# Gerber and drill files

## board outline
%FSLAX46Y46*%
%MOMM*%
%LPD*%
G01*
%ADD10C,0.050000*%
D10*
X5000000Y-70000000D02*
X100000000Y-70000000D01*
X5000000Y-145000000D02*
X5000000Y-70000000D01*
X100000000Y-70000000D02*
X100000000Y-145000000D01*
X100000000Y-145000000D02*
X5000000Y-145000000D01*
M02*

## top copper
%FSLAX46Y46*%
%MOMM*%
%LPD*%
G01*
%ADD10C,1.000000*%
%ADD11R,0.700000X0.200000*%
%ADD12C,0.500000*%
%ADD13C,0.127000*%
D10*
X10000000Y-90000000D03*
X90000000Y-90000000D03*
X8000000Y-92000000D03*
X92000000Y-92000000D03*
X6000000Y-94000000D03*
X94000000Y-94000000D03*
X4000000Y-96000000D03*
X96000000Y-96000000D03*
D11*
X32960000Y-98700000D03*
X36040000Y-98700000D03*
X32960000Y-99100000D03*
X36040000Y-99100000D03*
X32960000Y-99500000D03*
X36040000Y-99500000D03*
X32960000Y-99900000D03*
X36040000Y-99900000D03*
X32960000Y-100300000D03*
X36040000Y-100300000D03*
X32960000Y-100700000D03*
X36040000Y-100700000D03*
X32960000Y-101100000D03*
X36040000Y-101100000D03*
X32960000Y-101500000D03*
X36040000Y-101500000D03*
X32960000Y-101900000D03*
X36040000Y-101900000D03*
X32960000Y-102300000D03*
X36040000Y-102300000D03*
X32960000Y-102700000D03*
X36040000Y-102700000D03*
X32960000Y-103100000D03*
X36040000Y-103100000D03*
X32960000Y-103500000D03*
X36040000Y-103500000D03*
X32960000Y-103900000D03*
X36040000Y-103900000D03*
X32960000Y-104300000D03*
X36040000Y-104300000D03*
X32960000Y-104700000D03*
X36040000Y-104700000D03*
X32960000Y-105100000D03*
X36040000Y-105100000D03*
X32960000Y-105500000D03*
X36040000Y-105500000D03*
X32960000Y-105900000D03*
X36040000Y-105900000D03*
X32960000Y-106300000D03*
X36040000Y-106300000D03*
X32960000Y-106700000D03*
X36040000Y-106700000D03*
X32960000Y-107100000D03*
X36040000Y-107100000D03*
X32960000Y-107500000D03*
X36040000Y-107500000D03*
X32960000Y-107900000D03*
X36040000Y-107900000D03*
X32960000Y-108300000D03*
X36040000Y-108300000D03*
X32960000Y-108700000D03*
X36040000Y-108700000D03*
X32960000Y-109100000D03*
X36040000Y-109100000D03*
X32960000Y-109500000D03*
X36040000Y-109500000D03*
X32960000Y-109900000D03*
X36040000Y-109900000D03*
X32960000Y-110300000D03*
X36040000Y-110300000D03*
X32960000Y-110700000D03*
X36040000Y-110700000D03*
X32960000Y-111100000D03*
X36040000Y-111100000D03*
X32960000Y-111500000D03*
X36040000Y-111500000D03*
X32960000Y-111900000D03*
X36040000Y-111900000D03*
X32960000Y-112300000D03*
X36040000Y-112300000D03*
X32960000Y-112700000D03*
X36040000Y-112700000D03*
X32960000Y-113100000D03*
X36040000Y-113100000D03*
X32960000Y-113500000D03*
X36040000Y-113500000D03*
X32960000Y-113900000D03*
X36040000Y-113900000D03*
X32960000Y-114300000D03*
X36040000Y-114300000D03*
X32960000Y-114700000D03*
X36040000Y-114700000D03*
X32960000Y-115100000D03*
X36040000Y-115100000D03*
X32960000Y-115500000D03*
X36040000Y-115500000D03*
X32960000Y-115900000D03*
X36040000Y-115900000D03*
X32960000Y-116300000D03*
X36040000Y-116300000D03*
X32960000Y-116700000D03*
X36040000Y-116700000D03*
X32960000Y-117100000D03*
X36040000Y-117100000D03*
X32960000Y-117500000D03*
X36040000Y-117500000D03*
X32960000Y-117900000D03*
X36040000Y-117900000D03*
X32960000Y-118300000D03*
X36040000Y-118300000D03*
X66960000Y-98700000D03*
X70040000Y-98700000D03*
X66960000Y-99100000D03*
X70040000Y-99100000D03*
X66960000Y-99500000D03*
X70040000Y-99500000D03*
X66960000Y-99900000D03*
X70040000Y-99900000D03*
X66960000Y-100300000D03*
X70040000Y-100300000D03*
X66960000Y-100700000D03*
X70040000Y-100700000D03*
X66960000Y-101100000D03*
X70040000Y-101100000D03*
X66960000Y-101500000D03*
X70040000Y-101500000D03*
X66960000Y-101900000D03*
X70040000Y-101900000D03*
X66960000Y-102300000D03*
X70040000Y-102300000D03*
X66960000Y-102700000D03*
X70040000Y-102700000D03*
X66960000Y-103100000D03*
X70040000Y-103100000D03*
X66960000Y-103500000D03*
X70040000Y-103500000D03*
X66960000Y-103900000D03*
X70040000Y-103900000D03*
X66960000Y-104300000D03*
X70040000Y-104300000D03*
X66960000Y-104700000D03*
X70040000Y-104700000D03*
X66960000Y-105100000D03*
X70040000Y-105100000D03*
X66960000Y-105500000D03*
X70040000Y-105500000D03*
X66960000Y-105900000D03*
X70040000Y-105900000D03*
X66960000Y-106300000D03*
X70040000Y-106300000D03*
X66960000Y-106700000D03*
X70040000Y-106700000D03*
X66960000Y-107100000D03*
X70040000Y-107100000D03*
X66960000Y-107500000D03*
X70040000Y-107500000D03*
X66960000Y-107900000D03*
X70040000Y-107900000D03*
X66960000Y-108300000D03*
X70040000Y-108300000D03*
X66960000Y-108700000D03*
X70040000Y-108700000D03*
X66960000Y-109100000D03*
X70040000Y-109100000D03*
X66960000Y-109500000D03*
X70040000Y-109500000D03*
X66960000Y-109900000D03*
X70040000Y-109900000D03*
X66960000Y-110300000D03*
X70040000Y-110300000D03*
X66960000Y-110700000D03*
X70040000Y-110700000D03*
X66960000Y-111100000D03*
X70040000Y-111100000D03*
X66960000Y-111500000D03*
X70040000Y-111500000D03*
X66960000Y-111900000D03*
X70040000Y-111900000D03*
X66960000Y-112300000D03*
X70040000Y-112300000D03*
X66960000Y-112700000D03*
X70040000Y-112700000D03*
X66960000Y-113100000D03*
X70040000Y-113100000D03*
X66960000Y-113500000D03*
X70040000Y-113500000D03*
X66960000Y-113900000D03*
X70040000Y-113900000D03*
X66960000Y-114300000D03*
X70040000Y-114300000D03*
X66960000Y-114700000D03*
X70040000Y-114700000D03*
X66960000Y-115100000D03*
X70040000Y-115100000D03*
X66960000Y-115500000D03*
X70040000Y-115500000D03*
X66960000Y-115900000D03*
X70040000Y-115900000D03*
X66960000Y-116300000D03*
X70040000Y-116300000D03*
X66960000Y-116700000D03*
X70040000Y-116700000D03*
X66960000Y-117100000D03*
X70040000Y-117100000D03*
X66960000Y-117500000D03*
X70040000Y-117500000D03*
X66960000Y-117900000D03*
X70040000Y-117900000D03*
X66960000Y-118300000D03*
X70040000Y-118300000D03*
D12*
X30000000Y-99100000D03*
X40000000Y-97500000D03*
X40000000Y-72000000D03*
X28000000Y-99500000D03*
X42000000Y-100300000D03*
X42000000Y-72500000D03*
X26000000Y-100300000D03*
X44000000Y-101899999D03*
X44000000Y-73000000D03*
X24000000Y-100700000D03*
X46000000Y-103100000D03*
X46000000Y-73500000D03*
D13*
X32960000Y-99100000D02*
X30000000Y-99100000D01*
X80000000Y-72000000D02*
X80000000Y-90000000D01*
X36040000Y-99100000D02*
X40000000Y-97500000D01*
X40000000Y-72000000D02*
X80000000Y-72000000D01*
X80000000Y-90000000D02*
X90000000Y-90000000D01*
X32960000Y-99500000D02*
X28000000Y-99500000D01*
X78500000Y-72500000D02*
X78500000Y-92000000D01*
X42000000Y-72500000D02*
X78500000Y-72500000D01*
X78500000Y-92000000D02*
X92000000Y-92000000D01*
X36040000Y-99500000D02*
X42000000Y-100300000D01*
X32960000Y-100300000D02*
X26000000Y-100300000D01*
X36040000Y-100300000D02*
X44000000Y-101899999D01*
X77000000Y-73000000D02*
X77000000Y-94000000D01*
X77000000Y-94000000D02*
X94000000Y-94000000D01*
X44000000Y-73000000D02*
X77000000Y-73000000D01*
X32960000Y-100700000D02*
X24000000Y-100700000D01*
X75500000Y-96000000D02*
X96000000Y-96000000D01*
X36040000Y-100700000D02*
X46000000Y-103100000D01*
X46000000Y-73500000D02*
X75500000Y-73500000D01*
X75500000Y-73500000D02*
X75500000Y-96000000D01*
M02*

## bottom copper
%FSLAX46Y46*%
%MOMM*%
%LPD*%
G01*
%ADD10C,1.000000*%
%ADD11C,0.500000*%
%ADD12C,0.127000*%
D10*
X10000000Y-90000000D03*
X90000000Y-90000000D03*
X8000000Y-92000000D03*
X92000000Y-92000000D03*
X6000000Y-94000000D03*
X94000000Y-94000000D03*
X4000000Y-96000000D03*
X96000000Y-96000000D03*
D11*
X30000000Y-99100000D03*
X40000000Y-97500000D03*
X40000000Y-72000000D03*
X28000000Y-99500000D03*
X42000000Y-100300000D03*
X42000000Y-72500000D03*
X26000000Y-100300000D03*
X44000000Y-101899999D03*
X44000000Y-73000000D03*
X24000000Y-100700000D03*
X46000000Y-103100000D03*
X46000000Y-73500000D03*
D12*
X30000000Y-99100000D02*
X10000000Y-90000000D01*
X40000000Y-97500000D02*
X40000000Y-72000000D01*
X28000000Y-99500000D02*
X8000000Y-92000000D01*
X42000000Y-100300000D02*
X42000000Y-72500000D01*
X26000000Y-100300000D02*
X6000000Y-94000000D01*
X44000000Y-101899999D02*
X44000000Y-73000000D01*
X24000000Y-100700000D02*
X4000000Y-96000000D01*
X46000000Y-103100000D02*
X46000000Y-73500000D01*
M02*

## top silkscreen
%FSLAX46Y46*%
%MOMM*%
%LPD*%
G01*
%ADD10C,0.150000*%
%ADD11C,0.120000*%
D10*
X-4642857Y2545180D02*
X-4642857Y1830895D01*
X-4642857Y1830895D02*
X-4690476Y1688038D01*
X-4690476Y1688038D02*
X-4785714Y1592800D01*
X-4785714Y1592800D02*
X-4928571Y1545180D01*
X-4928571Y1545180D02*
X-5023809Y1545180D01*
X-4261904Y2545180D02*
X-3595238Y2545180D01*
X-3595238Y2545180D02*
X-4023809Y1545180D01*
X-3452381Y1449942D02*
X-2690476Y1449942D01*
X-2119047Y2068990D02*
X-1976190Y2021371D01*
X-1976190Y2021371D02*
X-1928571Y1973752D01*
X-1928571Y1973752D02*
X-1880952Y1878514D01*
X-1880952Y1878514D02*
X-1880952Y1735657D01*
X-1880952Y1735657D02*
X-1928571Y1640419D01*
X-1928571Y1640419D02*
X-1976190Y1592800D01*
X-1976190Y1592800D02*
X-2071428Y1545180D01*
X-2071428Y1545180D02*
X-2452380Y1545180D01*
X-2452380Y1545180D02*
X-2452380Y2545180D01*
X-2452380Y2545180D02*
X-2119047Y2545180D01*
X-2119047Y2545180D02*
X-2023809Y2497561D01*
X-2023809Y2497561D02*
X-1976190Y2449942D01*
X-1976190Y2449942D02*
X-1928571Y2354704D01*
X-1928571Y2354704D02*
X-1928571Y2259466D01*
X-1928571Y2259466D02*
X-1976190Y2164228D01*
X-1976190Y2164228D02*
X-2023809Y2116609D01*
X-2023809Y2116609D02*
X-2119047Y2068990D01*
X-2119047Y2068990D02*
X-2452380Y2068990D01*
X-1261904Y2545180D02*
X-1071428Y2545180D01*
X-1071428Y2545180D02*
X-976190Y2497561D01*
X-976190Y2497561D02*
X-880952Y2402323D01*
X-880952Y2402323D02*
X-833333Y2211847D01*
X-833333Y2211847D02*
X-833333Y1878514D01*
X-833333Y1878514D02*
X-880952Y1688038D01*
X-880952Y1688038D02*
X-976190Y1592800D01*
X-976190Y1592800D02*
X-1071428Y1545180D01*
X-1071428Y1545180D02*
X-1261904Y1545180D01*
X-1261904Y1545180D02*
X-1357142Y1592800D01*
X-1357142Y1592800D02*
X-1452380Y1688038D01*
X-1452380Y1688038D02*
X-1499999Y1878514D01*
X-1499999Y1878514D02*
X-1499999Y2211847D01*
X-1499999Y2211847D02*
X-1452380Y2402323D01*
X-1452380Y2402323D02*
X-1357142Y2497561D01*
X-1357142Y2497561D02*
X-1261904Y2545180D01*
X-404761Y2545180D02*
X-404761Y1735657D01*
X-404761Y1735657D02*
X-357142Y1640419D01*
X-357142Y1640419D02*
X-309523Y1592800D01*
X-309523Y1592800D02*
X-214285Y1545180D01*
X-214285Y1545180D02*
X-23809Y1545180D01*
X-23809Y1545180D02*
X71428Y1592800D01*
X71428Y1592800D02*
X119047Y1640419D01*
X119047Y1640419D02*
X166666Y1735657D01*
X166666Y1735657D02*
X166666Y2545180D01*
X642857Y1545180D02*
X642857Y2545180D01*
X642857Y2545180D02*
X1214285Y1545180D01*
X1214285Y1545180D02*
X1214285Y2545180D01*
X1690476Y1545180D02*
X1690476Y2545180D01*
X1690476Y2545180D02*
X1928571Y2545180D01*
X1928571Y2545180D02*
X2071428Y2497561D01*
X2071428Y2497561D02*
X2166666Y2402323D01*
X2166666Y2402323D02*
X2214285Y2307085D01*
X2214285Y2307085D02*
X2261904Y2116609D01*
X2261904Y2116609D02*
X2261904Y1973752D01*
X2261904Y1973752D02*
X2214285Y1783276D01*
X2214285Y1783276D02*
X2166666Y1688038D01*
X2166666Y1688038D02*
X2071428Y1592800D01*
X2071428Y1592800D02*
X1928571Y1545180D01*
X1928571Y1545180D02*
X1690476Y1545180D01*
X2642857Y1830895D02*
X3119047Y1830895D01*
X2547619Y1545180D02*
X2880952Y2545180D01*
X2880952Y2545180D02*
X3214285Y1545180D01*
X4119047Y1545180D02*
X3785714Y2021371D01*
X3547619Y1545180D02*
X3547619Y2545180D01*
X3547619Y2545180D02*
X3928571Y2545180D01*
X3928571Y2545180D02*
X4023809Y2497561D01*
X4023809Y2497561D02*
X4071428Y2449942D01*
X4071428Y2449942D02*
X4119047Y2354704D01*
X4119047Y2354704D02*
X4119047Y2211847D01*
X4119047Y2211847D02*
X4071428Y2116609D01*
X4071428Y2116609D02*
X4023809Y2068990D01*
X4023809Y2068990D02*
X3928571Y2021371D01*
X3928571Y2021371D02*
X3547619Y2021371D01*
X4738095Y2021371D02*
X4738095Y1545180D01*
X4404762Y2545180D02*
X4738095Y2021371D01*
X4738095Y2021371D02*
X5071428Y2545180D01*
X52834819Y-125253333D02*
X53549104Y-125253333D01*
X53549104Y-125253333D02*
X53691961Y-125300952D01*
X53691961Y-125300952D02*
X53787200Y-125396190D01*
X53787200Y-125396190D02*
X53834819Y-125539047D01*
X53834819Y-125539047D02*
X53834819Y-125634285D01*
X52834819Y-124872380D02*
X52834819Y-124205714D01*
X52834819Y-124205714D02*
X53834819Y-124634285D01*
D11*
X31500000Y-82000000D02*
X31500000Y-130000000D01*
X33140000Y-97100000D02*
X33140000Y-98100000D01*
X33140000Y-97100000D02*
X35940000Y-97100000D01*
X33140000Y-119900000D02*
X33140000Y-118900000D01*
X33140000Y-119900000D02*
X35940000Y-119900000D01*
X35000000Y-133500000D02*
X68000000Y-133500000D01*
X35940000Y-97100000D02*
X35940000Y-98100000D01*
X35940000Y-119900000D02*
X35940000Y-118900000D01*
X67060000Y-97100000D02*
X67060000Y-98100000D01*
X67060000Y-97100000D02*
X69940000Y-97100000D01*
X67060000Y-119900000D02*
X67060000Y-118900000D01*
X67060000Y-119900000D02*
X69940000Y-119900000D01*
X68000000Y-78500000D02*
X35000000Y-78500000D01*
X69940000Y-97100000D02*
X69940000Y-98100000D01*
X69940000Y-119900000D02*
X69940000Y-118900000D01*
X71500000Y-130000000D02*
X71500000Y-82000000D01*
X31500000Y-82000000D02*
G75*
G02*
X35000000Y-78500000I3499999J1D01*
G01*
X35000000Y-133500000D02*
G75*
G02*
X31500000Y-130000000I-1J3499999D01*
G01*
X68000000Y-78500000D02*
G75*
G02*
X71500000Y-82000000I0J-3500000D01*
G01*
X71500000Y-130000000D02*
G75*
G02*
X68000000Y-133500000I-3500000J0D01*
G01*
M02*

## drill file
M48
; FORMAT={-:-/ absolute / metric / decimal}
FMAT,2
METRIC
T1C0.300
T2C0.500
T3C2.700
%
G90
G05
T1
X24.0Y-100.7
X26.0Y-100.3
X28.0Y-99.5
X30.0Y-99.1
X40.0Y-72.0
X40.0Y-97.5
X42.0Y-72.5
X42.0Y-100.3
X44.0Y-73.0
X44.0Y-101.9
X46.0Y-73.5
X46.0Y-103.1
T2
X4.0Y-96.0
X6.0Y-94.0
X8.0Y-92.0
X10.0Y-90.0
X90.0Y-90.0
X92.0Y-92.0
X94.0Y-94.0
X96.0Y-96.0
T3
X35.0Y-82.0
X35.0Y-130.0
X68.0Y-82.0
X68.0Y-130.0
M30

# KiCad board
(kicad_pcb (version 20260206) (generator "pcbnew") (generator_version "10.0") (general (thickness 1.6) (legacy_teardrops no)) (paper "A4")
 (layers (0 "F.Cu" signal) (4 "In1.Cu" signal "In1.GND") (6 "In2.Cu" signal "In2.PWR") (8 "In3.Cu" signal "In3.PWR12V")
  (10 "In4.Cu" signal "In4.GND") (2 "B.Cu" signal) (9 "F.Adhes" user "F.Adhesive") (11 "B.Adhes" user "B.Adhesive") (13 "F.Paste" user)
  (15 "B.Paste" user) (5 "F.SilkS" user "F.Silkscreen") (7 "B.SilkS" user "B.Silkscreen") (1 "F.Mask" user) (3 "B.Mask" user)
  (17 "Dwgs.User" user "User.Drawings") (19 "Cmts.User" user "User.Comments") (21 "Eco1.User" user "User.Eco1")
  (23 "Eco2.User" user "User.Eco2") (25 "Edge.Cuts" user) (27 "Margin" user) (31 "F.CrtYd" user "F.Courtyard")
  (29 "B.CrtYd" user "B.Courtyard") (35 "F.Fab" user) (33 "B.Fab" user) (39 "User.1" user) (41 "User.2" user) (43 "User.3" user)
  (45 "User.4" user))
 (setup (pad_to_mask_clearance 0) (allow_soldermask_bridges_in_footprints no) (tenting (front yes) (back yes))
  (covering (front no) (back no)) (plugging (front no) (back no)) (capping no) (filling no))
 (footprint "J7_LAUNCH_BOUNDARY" (layer "F.Cu") (at 0 0)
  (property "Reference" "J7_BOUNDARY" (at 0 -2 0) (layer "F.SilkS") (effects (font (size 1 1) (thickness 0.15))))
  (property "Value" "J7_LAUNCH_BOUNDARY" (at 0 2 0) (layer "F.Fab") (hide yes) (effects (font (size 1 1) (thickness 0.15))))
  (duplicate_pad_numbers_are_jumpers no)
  (pad "3" thru_hole circle (at 10 90) (size 1 1) (drill 0.5) (layers "*.Cu" "*.Mask") (remove_unused_layers no) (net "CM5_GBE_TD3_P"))
  (pad "4" thru_hole circle (at 90 90) (size 1 1) (drill 0.5) (layers "*.Cu" "*.Mask") (remove_unused_layers no) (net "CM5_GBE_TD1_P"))
  (pad "5" thru_hole circle (at 8 92) (size 1 1) (drill 0.5) (layers "*.Cu" "*.Mask") (remove_unused_layers no) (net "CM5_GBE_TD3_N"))
  (pad "6" thru_hole circle (at 92 92) (size 1 1) (drill 0.5) (layers "*.Cu" "*.Mask") (remove_unused_layers no) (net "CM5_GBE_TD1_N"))
  (pad "9" thru_hole circle (at 6 94) (size 1 1) (drill 0.5) (layers "*.Cu" "*.Mask") (remove_unused_layers no) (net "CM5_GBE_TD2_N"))
  (pad "10" thru_hole circle (at 94 94) (size 1 1) (drill 0.5) (layers "*.Cu" "*.Mask") (remove_unused_layers no) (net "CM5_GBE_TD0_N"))
  (pad "11" thru_hole circle (at 4 96) (size 1 1) (drill 0.5) (layers "*.Cu" "*.Mask") (remove_unused_layers no) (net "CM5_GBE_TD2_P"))
  (pad "12" thru_hole circle (at 96 96) (size 1 1) (drill 0.5) (layers "*.Cu" "*.Mask") (remove_unused_layers no) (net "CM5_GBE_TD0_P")))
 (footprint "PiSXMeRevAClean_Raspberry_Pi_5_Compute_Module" (layer "B.Cu") (at 35 130)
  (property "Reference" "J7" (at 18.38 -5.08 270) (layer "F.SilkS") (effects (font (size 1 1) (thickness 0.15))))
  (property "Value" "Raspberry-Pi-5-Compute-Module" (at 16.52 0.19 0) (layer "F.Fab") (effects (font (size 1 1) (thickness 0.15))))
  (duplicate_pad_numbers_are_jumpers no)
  (fp_line (start -3.5 -48) (end -3.5 0) (stroke (width 0.12) (type solid)) (layer "F.SilkS"))
  (fp_line (start -1.86 -32.9) (end -1.86 -31.9) (stroke (width 0.12) (type solid)) (layer "F.SilkS"))
  (fp_line (start -1.86 -32.9) (end 0.94 -32.9) (stroke (width 0.12) (type solid)) (layer "F.SilkS"))
  (fp_line (start -1.86 -10.1) (end -1.86 -11.1) (stroke (width 0.12) (type solid)) (layer "F.SilkS"))
  (fp_line (start -1.86 -10.1) (end 0.94 -10.1) (stroke (width 0.12) (type solid)) (layer "F.SilkS"))
  (fp_line (start 0 3.5) (end 33 3.5) (stroke (width 0.12) (type solid)) (layer "F.SilkS"))
  (fp_line (start 0.94 -32.9) (end 0.94 -31.9) (stroke (width 0.12) (type solid)) (layer "F.SilkS"))
  (fp_line (start 0.94 -10.1) (end 0.94 -11.1) (stroke (width 0.12) (type solid)) (layer "F.SilkS"))
  (fp_line (start 32.06 -32.9) (end 32.06 -31.9) (stroke (width 0.12) (type solid)) (layer "F.SilkS"))
  (fp_line (start 32.06 -32.9) (end 34.94 -32.9) (stroke (width 0.12) (type solid)) (layer "F.SilkS"))
  (fp_line (start 32.06 -10.1) (end 32.06 -11.1) (stroke (width 0.12) (type solid)) (layer "F.SilkS"))
  (fp_line (start 32.06 -10.1) (end 34.94 -10.1) (stroke (width 0.12) (type solid)) (layer "F.SilkS"))
  (fp_line (start 33 -51.5) (end 0 -51.5) (stroke (width 0.12) (type solid)) (layer "F.SilkS"))
  (fp_line (start 34.94 -32.9) (end 34.94 -31.9) (stroke (width 0.12) (type solid)) (layer "F.SilkS"))
  (fp_line (start 34.94 -10.1) (end 34.94 -11.1) (stroke (width 0.12) (type solid)) (layer "F.SilkS"))
  (fp_line (start 36.5 0) (end 36.5 -48) (stroke (width 0.12) (type solid)) (layer "F.SilkS"))
  (fp_arc (start -3.5 -48) (mid -2.474874 -50.474874) (end 0 -51.5) (stroke (width 0.12) (type solid)) (layer "F.SilkS"))
  (fp_arc (start 0 3.5) (mid -2.474874 2.474874) (end -3.5 0) (stroke (width 0.12) (type solid)) (layer "F.SilkS"))
  (fp_arc (start 33 -51.5) (mid 35.474874 -50.474874) (end 36.5 -48) (stroke (width 0.12) (type solid)) (layer "F.SilkS"))
  (fp_arc (start 36.5 0) (mid 35.474874 2.474874) (end 33 3.5) (stroke (width 0.12) (type solid)) (layer "F.SilkS"))
  (pad "" np_thru_hole circle (at 0 -48) (size 2.7 2.7) (drill 2.7) (layers "*.Cu" "*.Mask") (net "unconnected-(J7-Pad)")
   (solder_mask_margin 1.7) (clearance 1.7))
  (pad "" np_thru_hole circle (at 0 0) (size 2.7 2.7) (drill 2.7) (layers "*.Cu" "*.Mask") (solder_mask_margin 1.7) (clearance 1.7))
  (pad "" np_thru_hole circle (at 33 -48) (size 2.7 2.7) (drill 2.7) (layers "*.Cu" "*.Mask") (solder_mask_margin 1.7) (clearance 1.7))
  (pad "" np_thru_hole circle (at 33 0) (size 2.7 2.7) (drill 2.7) (layers "*.Cu" "*.Mask") (solder_mask_margin 1.7) (clearance 1.7))
  (pad "1" smd rect (at -2.04 -31.3 270) (size 0.2 0.7) (layers "F.Cu" "F.Mask" "F.Paste") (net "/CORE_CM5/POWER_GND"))
  (pad "2" smd rect (at 1.04 -31.3 270) (size 0.2 0.7) (layers "F.Cu" "F.Mask" "F.Paste") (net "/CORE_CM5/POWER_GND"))
  (pad "3" smd rect (at -2.04 -30.9 270) (size 0.2 0.7) (layers "F.Cu" "F.Mask" "F.Paste") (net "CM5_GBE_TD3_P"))
  (pad "4" smd rect (at 1.04 -30.9 270) (size 0.2 0.7) (layers "F.Cu" "F.Mask" "F.Paste") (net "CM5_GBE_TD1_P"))
  (pad "5" smd rect (at -2.04 -30.5 270) (size 0.2 0.7) (layers "F.Cu" "F.Mask" "F.Paste") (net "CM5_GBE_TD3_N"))
  (pad "6" smd rect (at 1.04 -30.5 270) (size 0.2 0.7) (layers "F.Cu" "F.Mask" "F.Paste") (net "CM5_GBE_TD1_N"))
  (pad "7" smd rect (at -2.04 -30.1 270) (size 0.2 0.7) (layers "F.Cu" "F.Mask" "F.Paste") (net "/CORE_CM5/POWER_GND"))
  (pad "8" smd rect (at 1.04 -30.1 270) (size 0.2 0.7) (layers "F.Cu" "F.Mask" "F.Paste") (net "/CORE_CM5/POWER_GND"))
  (pad "9" smd rect (at -2.04 -29.7 270) (size 0.2 0.7) (layers "F.Cu" "F.Mask" "F.Paste") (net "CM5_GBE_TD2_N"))
  (pad "10" smd rect (at 1.04 -29.7 270) (size 0.2 0.7) (layers "F.Cu" "F.Mask" "F.Paste") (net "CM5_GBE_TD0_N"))
  (pad "11" smd rect (at -2.04 -29.3 270) (size 0.2 0.7) (layers "F.Cu" "F.Mask" "F.Paste") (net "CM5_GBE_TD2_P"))
  (pad "12" smd rect (at 1.04 -29.3 270) (size 0.2 0.7) (layers "F.Cu" "F.Mask" "F.Paste") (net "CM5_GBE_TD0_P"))
  (pad "13" smd rect (at -2.04 -28.9 270) (size 0.2 0.7) (layers "F.Cu" "F.Mask" "F.Paste") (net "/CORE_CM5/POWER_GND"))
  (pad "14" smd rect (at 1.04 -28.9 270) (size 0.2 0.7) (layers "F.Cu" "F.Mask" "F.Paste") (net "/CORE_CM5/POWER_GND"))
  (pad "15" smd rect (at -2.04 -28.5 270) (size 0.2 0.7) (layers "F.Cu" "F.Mask" "F.Paste")
   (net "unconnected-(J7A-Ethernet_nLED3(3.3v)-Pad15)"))
  (pad "16" smd rect (at 1.04 -28.5 270) (size 0.2 0.7) (layers "F.Cu" "F.Mask" "F.Paste") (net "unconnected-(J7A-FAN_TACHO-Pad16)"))
  (pad "17" smd rect (at -2.04 -28.1 270) (size 0.2 0.7) (layers "F.Cu" "F.Mask" "F.Paste")
   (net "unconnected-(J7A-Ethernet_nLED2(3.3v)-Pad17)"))
  (pad "18" smd rect (at 1.04 -28.1 270) (size 0.2 0.7) (layers "F.Cu" "F.Mask" "F.Paste")
   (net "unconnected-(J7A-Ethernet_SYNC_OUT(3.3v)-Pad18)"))
  (pad "19" smd rect (at -2.04 -27.7 270) (size 0.2 0.7) (layers "F.Cu" "F.Mask" "F.Paste") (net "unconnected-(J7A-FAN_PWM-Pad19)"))
  (pad "20" smd rect (at 1.04 -27.7 270) (size 0.2 0.7) (layers "F.Cu" "F.Mask" "F.Paste") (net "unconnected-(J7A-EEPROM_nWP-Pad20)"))
  (pad "21" smd rect (at -2.04 -27.3 270) (size 0.2 0.7) (layers "F.Cu" "F.Mask" "F.Paste") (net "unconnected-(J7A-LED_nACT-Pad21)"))
  (pad "22" smd rect (at 1.04 -27.3 270) (size 0.2 0.7) (layers "F.Cu" "F.Mask" "F.Paste") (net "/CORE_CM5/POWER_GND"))
  (pad "23" smd rect (at -2.04 -26.9 270) (size 0.2 0.7) (layers "F.Cu" "F.Mask" "F.Paste") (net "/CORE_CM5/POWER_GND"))
  (pad "24" smd rect (at 1.04 -26.9 270) (size 0.2 0.7) (layers "F.Cu" "F.Mask" "F.Paste") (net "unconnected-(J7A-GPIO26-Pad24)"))
  (pad "25" smd rect (at -2.04 -26.5 270) (size 0.2 0.7) (layers "F.Cu" "F.Mask" "F.Paste") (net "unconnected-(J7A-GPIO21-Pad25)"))
  (pad "26" smd rect (at 1.04 -26.5 270) (size 0.2 0.7) (layers "F.Cu" "F.Mask" "F.Paste") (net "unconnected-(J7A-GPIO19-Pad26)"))
  (pad "27" smd rect (at -2.04 -26.1 270) (size 0.2 0.7) (layers "F.Cu" "F.Mask" "F.Paste") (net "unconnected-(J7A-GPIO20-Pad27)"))
  (pad "28" smd rect (at 1.04 -26.1 270) (size 0.2 0.7) (layers "F.Cu" "F.Mask" "F.Paste") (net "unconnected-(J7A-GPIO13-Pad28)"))
  (pad "29" smd rect (at -2.04 -25.7 270) (size 0.2 0.7) (layers "F.Cu" "F.Mask" "F.Paste") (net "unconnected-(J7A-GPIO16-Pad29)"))
  (pad "30" smd rect (at 1.04 -25.7 270) (size 0.2 0.7) (layers "F.Cu" "F.Mask" "F.Paste") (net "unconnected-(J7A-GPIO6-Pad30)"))
  (pad "31" smd rect (at -2.04 -25.3 270) (size 0.2 0.7) (layers "F.Cu" "F.Mask" "F.Paste") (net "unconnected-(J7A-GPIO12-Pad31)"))
  (pad "32" smd rect (at 1.04 -25.3 270) (size 0.2 0.7) (layers "F.Cu" "F.Mask" "F.Paste") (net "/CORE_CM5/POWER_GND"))
  (pad "33" smd rect (at -2.04 -24.9 270) (size 0.2 0.7) (layers "F.Cu" "F.Mask" "F.Paste") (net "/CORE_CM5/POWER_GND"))
  (pad "34" smd rect (at 1.04 -24.9 270) (size 0.2 0.7) (layers "F.Cu" "F.Mask" "F.Paste") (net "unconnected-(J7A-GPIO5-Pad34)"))
  (pad "35" smd rect (at -2.04 -24.5 270) (size 0.2 0.7) (layers "F.Cu" "F.Mask" "F.Paste") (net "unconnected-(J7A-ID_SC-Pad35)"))
  (pad "36" smd rect (at 1.04 -24.5 270) (size 0.2 0.7) (layers "F.Cu" "F.Mask" "F.Paste") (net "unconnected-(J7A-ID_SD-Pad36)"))
  (pad "37" smd rect (at -2.04 -24.1 270) (size 0.2 0.7) (layers "F.Cu" "F.Mask" "F.Paste") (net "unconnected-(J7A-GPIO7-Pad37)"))
  (pad "38" smd rect (at 1.04 -24.1 270) (size 0.2 0.7) (layers "F.Cu" "F.Mask" "F.Paste") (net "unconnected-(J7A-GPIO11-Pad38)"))
  (pad "39" smd rect (at -2.04 -23.7 270) (size 0.2 0.7) (layers "F.Cu" "F.Mask" "F.Paste") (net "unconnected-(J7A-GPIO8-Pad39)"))
  (pad "40" smd rect (at 1.04 -23.7 270) (size 0.2 0.7) (layers "F.Cu" "F.Mask" "F.Paste") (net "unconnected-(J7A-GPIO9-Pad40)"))
  (pad "41" smd rect (at -2.04 -23.3 270) (size 0.2 0.7) (layers "F.Cu" "F.Mask" "F.Paste") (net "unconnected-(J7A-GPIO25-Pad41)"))
  (pad "42" smd rect (at 1.04 -23.3 270) (size 0.2 0.7) (layers "F.Cu" "F.Mask" "F.Paste") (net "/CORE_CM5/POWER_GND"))
  (pad "43" smd rect (at -2.04 -22.9 270) (size 0.2 0.7) (layers "F.Cu" "F.Mask" "F.Paste") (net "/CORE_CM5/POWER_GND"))
  (pad "44" smd rect (at 1.04 -22.9 270) (size 0.2 0.7) (layers "F.Cu" "F.Mask" "F.Paste") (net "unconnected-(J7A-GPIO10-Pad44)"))
  (pad "45" smd rect (at -2.04 -22.5 270) (size 0.2 0.7) (layers "F.Cu" "F.Mask" "F.Paste") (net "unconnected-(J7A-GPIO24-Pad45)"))
  (pad "46" smd rect (at 1.04 -22.5 270) (size 0.2 0.7) (layers "F.Cu" "F.Mask" "F.Paste") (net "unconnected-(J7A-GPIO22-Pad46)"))
  (pad "47" smd rect (at -2.04 -22.1 270) (size 0.2 0.7) (layers "F.Cu" "F.Mask" "F.Paste") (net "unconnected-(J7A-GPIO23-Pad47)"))
  (pad "48" smd rect (at 1.04 -22.1 270) (size 0.2 0.7) (layers "F.Cu" "F.Mask" "F.Paste") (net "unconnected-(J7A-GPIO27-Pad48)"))
  (pad "49" smd rect (at -2.04 -21.7 270) (size 0.2 0.7) (layers "F.Cu" "F.Mask" "F.Paste") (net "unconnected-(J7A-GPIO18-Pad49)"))
  (pad "50" smd rect (at 1.04 -21.7 270) (size 0.2 0.7) (layers "F.Cu" "F.Mask" "F.Paste") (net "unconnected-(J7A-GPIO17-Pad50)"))
  (pad "51" smd rect (at -2.04 -21.3 270) (size 0.2 0.7) (layers "F.Cu" "F.Mask" "F.Paste") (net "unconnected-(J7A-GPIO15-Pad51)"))
  (pad "52" smd rect (at 1.04 -21.3 270) (size 0.2 0.7) (layers "F.Cu" "F.Mask" "F.Paste") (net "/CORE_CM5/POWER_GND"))
  (pad "53" smd rect (at -2.04 -20.9 270) (size 0.2 0.7) (layers "F.Cu" "F.Mask" "F.Paste") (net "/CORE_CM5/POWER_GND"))
  (pad "54" smd rect (at 1.04 -20.9 270) (size 0.2 0.7) (layers "F.Cu" "F.Mask" "F.Paste") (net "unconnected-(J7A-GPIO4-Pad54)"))
  (pad "55" smd rect (at -2.04 -20.5 270) (size 0.2 0.7) (layers "F.Cu" "F.Mask" "F.Paste") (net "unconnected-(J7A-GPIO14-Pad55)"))
  (pad "56" smd rect (at 1.04 -20.5 270) (size 0.2 0.7) (layers "F.Cu" "F.Mask" "F.Paste") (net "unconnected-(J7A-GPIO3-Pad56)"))
  (pad "57" smd rect (at -2.04 -20.1 270) (size 0.2 0.7) (layers "F.Cu" "F.Mask" "F.Paste") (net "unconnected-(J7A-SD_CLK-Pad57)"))
  (pad "58" smd rect (at 1.04 -20.1 270) (size 0.2 0.7) (layers "F.Cu" "F.Mask" "F.Paste") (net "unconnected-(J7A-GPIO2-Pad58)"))
  (pad "59" smd rect (at -2.04 -19.7 270) (size 0.2 0.7) (layers "F.Cu" "F.Mask" "F.Paste") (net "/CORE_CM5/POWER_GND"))
  (pad "60" smd rect (at 1.04 -19.7 270) (size 0.2 0.7) (layers "F.Cu" "F.Mask" "F.Paste") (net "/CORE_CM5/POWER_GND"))
  (pad "61" smd rect (at -2.04 -19.3 270) (size 0.2 0.7) (layers "F.Cu" "F.Mask" "F.Paste") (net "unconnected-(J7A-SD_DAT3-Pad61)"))
  (pad "62" smd rect (at 1.04 -19.3 270) (size 0.2 0.7) (layers "F.Cu" "F.Mask" "F.Paste") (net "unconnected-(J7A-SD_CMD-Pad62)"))
  (pad "63" smd rect (at -2.04 -18.9 270) (size 0.2 0.7) (layers "F.Cu" "F.Mask" "F.Paste") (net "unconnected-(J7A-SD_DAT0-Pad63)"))
  (pad "64" smd rect (at 1.04 -18.9 270) (size 0.2 0.7) (layers "F.Cu" "F.Mask" "F.Paste") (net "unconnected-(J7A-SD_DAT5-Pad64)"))
  (pad "65" smd rect (at -2.04 -18.5 270) (size 0.2 0.7) (layers "F.Cu" "F.Mask" "F.Paste") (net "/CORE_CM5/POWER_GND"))
  (pad "66" smd rect (at 1.04 -18.5 270) (size 0.2 0.7) (layers "F.Cu" "F.Mask" "F.Paste") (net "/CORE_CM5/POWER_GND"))
  (pad "67" smd rect (at -2.04 -18.1 270) (size 0.2 0.7) (layers "F.Cu" "F.Mask" "F.Paste") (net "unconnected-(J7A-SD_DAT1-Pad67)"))
  (pad "68" smd rect (at 1.04 -18.1 270) (size 0.2 0.7) (layers "F.Cu" "F.Mask" "F.Paste") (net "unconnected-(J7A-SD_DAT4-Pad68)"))
  (pad "69" smd rect (at -2.04 -17.7 270) (size 0.2 0.7) (layers "F.Cu" "F.Mask" "F.Paste") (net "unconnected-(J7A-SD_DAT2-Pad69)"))
  (pad "70" smd rect (at 1.04 -17.7 270) (size 0.2 0.7) (layers "F.Cu" "F.Mask" "F.Paste") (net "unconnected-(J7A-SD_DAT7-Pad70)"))
  (pad "71" smd rect (at -2.04 -17.3 270) (size 0.2 0.7) (layers "F.Cu" "F.Mask" "F.Paste") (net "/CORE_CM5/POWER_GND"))
  (pad "72" smd rect (at 1.04 -17.3 270) (size 0.2 0.7) (layers "F.Cu" "F.Mask" "F.Paste") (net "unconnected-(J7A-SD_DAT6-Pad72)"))
  (pad "73" smd rect (at -2.04 -16.9 270) (size 0.2 0.7) (layers "F.Cu" "F.Mask" "F.Paste") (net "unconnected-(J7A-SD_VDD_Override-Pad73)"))
  (pad "74" smd rect (at 1.04 -16.9 270) (size 0.2 0.7) (layers "F.Cu" "F.Mask" "F.Paste") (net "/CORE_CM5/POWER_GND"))
  (pad "75" smd rect (at -2.04 -16.5 270) (size 0.2 0.7) (layers "F.Cu" "F.Mask" "F.Paste") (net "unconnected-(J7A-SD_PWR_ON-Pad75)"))
  (pad "76" smd rect (at 1.04 -16.5 270) (size 0.2 0.7) (layers "F.Cu" "F.Mask" "F.Paste") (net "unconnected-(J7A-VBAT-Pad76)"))
  (pad "77" smd rect (at -2.04 -16.1 270) (size 0.2 0.7) (layers "F.Cu" "F.Mask" "F.Paste") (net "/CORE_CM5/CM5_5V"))
  (pad "78" smd rect (at 1.04 -16.1 270) (size 0.2 0.7) (layers "F.Cu" "F.Mask" "F.Paste")
   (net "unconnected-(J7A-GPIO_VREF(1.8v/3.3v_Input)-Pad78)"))
  (pad "79" smd rect (at -2.04 -15.7 270) (size 0.2 0.7) (layers "F.Cu" "F.Mask" "F.Paste") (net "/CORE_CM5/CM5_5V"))
  (pad "80" smd rect (at 1.04 -15.7 270) (size 0.2 0.7) (layers "F.Cu" "F.Mask" "F.Paste") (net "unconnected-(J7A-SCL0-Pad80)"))
  (pad "81" smd rect (at -2.04 -15.3 270) (size 0.2 0.7) (layers "F.Cu" "F.Mask" "F.Paste") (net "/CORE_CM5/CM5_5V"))
  (pad "82" smd rect (at 1.04 -15.3 270) (size 0.2 0.7) (layers "F.Cu" "F.Mask" "F.Paste") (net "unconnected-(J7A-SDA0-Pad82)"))
  (pad "83" smd rect (at -2.04 -14.9 270) (size 0.2 0.7) (layers "F.Cu" "F.Mask" "F.Paste") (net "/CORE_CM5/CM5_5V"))
  (pad "84" smd rect (at 1.04 -14.9 270) (size 0.2 0.7) (layers "F.Cu" "F.Mask" "F.Paste") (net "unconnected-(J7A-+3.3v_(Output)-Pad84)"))
  (pad "85" smd rect (at -2.04 -14.5 270) (size 0.2 0.7) (layers "F.Cu" "F.Mask" "F.Paste") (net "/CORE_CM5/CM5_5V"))
  (pad "86" smd rect (at 1.04 -14.5 270) (size 0.2 0.7) (layers "F.Cu" "F.Mask" "F.Paste") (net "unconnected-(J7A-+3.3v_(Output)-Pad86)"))
  (pad "87" smd rect (at -2.04 -14.1 270) (size 0.2 0.7) (layers "F.Cu" "F.Mask" "F.Paste") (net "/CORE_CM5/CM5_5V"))
  (pad "88" smd rect (at 1.04 -14.1 270) (size 0.2 0.7) (layers "F.Cu" "F.Mask" "F.Paste") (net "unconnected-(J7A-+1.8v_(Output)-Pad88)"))
  (pad "89" smd rect (at -2.04 -13.7 270) (size 0.2 0.7) (layers "F.Cu" "F.Mask" "F.Paste") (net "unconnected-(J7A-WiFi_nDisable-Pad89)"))
  (pad "90" smd rect (at 1.04 -13.7 270) (size 0.2 0.7) (layers "F.Cu" "F.Mask" "F.Paste") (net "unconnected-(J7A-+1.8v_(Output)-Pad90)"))
  (pad "91" smd rect (at -2.04 -13.3 270) (size 0.2 0.7) (layers "F.Cu" "F.Mask" "F.Paste") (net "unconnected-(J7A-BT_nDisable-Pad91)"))
  (pad "92" smd rect (at 1.04 -13.3 270) (size 0.2 0.7) (layers "F.Cu" "F.Mask" "F.Paste") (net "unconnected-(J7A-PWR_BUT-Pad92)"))
  (pad "93" smd rect (at -2.04 -12.9 270) (size 0.2 0.7) (layers "F.Cu" "F.Mask" "F.Paste") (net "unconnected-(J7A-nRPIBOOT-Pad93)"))
  (pad "94" smd rect (at 1.04 -12.9 270) (size 0.2 0.7) (layers "F.Cu" "F.Mask" "F.Paste") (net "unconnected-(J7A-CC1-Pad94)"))
  (pad "95" smd rect (at -2.04 -12.5 270) (size 0.2 0.7) (layers "F.Cu" "F.Mask" "F.Paste") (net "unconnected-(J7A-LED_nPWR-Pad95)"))
  (pad "96" smd rect (at 1.04 -12.5 270) (size 0.2 0.7) (layers "F.Cu" "F.Mask" "F.Paste") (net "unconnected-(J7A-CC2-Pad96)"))
  (pad "97" smd rect (at -2.04 -12.1 270) (size 0.2 0.7) (layers "F.Cu" "F.Mask" "F.Paste") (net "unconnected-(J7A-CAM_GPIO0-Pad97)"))
  (pad "98" smd rect (at 1.04 -12.1 270) (size 0.2 0.7) (layers "F.Cu" "F.Mask" "F.Paste") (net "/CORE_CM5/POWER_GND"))
  (pad "99" smd rect (at -2.04 -11.7 270) (size 0.2 0.7) (layers "F.Cu" "F.Mask" "F.Paste") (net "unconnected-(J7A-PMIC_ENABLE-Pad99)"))
  (pad "100" smd rect (at 1.04 -11.7 270) (size 0.2 0.7) (layers "F.Cu" "F.Mask" "F.Paste") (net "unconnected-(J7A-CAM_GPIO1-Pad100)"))
  (pad "101" smd rect (at 31.96 -31.3 270) (size 0.2 0.7) (layers "F.Cu" "F.Mask" "F.Paste") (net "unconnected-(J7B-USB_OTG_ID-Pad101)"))
  (pad "102" smd rect (at 35.04 -31.3 270) (size 0.2 0.7) (layers "F.Cu" "F.Mask" "F.Paste") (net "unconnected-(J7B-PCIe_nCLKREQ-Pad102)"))
  (pad "103" smd rect (at 31.96 -30.9 270) (size 0.2 0.7) (layers "F.Cu" "F.Mask" "F.Paste") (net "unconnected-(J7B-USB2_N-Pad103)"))
  (pad "104" smd rect (at 35.04 -30.9 270) (size 0.2 0.7) (layers "F.Cu" "F.Mask" "F.Paste") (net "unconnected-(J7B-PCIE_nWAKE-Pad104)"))
  (pad "105" smd rect (at 31.96 -30.5 270) (size 0.2 0.7) (layers "F.Cu" "F.Mask" "F.Paste") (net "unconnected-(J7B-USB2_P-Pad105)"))
  (pad "106" smd rect (at 35.04 -30.5 270) (size 0.2 0.7) (layers "F.Cu" "F.Mask" "F.Paste") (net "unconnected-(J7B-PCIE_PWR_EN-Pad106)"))
  (pad "107" smd rect (at 31.96 -30.1 270) (size 0.2 0.7) (layers "F.Cu" "F.Mask" "F.Paste") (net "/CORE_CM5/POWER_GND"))
  (pad "108" smd rect (at 35.04 -30.1 270) (size 0.2 0.7) (layers "F.Cu" "F.Mask" "F.Paste") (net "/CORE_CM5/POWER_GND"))
  (pad "109" smd rect (at 31.96 -29.7 270) (size 0.2 0.7) (layers "F.Cu" "F.Mask" "F.Paste") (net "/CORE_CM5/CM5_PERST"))
  (pad "110" smd rect (at 35.04 -29.7 270) (size 0.2 0.7) (layers "F.Cu" "F.Mask" "F.Paste") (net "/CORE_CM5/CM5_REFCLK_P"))
  (pad "111" smd rect (at 31.96 -29.3 270) (size 0.2 0.7) (layers "F.Cu" "F.Mask" "F.Paste") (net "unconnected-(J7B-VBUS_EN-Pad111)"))
  (pad "112" smd rect (at 35.04 -29.3 270) (size 0.2 0.7) (layers "F.Cu" "F.Mask" "F.Paste") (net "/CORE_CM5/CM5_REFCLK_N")
   (die_length 0.01))
  (pad "113" smd rect (at 31.96 -28.9 270) (size 0.2 0.7) (layers "F.Cu" "F.Mask" "F.Paste") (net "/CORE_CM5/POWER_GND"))
  (pad "114" smd rect (at 35.04 -28.9 270) (size 0.2 0.7) (layers "F.Cu" "F.Mask" "F.Paste") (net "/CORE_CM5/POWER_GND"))
  (pad "115" smd rect (at 31.96 -28.5 270) (size 0.2 0.7) (layers "F.Cu" "F.Mask" "F.Paste") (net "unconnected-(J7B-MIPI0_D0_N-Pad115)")
   (die_length 0.01))
  (pad "116" smd rect (at 35.04 -28.5 270) (size 0.2 0.7) (layers "F.Cu" "F.Mask" "F.Paste") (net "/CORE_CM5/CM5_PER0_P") (die_length 0.84))
  (pad "117" smd rect (at 31.96 -28.1 270) (size 0.2 0.7) (layers "F.Cu" "F.Mask" "F.Paste") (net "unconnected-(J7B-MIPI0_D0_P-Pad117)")
   (die_length 0.02))
  (pad "118" smd rect (at 35.04 -28.1 270) (size 0.2 0.7) (layers "F.Cu" "F.Mask" "F.Paste") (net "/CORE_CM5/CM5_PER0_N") (die_length 0.84))
  (pad "119" smd rect (at 31.96 -27.7 270) (size 0.2 0.7) (layers "F.Cu" "F.Mask" "F.Paste") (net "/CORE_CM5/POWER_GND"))
  (pad "120" smd rect (at 35.04 -27.7 270) (size 0.2 0.7) (layers "F.Cu" "F.Mask" "F.Paste") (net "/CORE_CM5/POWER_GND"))
  (pad "121" smd rect (at 31.96 -27.3 270) (size 0.2 0.7) (layers "F.Cu" "F.Mask" "F.Paste") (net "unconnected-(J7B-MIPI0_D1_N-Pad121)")
   (die_length 0.4))
  (pad "122" smd rect (at 35.04 -27.3 270) (size 0.2 0.7) (layers "F.Cu" "F.Mask" "F.Paste") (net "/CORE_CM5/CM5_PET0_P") (die_length 3.71))
  (pad "123" smd rect (at 31.96 -26.9 270) (size 0.2 0.7) (layers "F.Cu" "F.Mask" "F.Paste") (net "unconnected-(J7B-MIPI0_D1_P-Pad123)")
   (die_length 0.4))
  (pad "124" smd rect (at 35.04 -26.9 270) (size 0.2 0.7) (layers "F.Cu" "F.Mask" "F.Paste") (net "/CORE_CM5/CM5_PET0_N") (die_length 3.72))
  (pad "125" smd rect (at 31.96 -26.5 270) (size 0.2 0.7) (layers "F.Cu" "F.Mask" "F.Paste") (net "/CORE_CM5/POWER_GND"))
  (pad "126" smd rect (at 35.04 -26.5 270) (size 0.2 0.7) (layers "F.Cu" "F.Mask" "F.Paste") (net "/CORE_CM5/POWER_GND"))
  (pad "127" smd rect (at 31.96 -26.1 270) (size 0.2 0.7) (layers "F.Cu" "F.Mask" "F.Paste") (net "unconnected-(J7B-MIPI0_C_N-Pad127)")
   (die_length 0.78))
  (pad "128" smd rect (at 35.04 -26.1 270) (size 0.2 0.7) (layers "F.Cu" "F.Mask" "F.Paste") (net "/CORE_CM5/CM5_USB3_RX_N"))
  (pad "129" smd rect (at 31.96 -25.7 270) (size 0.2 0.7) (layers "F.Cu" "F.Mask" "F.Paste") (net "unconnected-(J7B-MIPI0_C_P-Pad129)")
   (die_length 0.78))
  (pad "130" smd rect (at 35.04 -25.7 270) (size 0.2 0.7) (layers "F.Cu" "F.Mask" "F.Paste") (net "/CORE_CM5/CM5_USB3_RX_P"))
  (pad "131" smd rect (at 31.96 -25.3 270) (size 0.2 0.7) (layers "F.Cu" "F.Mask" "F.Paste") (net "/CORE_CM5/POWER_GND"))
  (pad "132" smd rect (at 35.04 -25.3 270) (size 0.2 0.7) (layers "F.Cu" "F.Mask" "F.Paste") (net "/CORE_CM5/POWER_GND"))
  (pad "133" smd rect (at 31.96 -24.9 270) (size 0.2 0.7) (layers "F.Cu" "F.Mask" "F.Paste") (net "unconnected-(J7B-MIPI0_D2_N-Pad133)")
   (die_length 0.04))
  (pad "134" smd rect (at 35.04 -24.9 270) (size 0.2 0.7) (layers "F.Cu" "F.Mask" "F.Paste") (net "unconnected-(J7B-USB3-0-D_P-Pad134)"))
  (pad "135" smd rect (at 31.96 -24.5 270) (size 0.2 0.7) (layers "F.Cu" "F.Mask" "F.Paste") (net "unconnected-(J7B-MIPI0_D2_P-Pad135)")
   (die_length 0.03))
  (pad "136" smd rect (at 35.04 -24.5 270) (size 0.2 0.7) (layers "F.Cu" "F.Mask" "F.Paste") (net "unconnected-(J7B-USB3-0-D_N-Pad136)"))
  (pad "137" smd rect (at 31.96 -24.1 270) (size 0.2 0.7) (layers "F.Cu" "F.Mask" "F.Paste") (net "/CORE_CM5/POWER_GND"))
  (pad "138" smd rect (at 35.04 -24.1 270) (size 0.2 0.7) (layers "F.Cu" "F.Mask" "F.Paste") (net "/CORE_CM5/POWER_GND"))
  (pad "139" smd rect (at 31.96 -23.7 270) (size 0.2 0.7) (layers "F.Cu" "F.Mask" "F.Paste") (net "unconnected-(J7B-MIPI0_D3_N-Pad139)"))
  (pad "140" smd rect (at 35.04 -23.7 270) (size 0.2 0.7) (layers "F.Cu" "F.Mask" "F.Paste") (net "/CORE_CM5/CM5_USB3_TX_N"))
  (pad "141" smd rect (at 31.96 -23.3 270) (size 0.2 0.7) (layers "F.Cu" "F.Mask" "F.Paste") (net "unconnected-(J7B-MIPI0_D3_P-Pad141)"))
  (pad "142" smd rect (at 35.04 -23.3 270) (size 0.2 0.7) (layers "F.Cu" "F.Mask" "F.Paste") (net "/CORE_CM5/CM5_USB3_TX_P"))
  (pad "143" smd rect (at 31.96 -22.9 270) (size 0.2 0.7) (layers "F.Cu" "F.Mask" "F.Paste") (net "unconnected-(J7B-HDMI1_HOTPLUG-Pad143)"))
  (pad "144" smd rect (at 35.04 -22.9 270) (size 0.2 0.7) (layers "F.Cu" "F.Mask" "F.Paste") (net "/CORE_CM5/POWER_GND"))
  (pad "145" smd rect (at 31.96 -22.5 270) (size 0.2 0.7) (layers "F.Cu" "F.Mask" "F.Paste") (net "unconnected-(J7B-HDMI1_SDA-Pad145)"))
  (pad "146" smd rect (at 35.04 -22.5 270) (size 0.2 0.7) (layers "F.Cu" "F.Mask" "F.Paste") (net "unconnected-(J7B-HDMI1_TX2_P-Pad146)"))
  (pad "147" smd rect (at 31.96 -22.1 270) (size 0.2 0.7) (layers "F.Cu" "F.Mask" "F.Paste") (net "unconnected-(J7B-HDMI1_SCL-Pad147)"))
  (pad "148" smd rect (at 35.04 -22.1 270) (size 0.2 0.7) (layers "F.Cu" "F.Mask" "F.Paste") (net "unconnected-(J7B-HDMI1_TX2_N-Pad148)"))
  (pad "149" smd rect (at 31.96 -21.7 270) (size 0.2 0.7) (layers "F.Cu" "F.Mask" "F.Paste") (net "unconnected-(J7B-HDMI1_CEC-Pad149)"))
  (pad "150" smd rect (at 35.04 -21.7 270) (size 0.2 0.7) (layers "F.Cu" "F.Mask" "F.Paste") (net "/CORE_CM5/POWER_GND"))
  (pad "151" smd rect (at 31.96 -21.3 270) (size 0.2 0.7) (layers "F.Cu" "F.Mask" "F.Paste") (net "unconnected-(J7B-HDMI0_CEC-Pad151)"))
  (pad "152" smd rect (at 35.04 -21.3 270) (size 0.2 0.7) (layers "F.Cu" "F.Mask" "F.Paste") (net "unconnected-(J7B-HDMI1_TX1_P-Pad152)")
   (die_length 5.18))
  (pad "153" smd rect (at 31.96 -20.9 270) (size 0.2 0.7) (layers "F.Cu" "F.Mask" "F.Paste") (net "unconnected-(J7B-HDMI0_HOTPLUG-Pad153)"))
  (pad "154" smd rect (at 35.04 -20.9 270) (size 0.2 0.7) (layers "F.Cu" "F.Mask" "F.Paste") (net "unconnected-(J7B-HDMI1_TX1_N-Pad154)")
   (die_length 5.18))
  (pad "155" smd rect (at 31.96 -20.5 270) (size 0.2 0.7) (layers "F.Cu" "F.Mask" "F.Paste") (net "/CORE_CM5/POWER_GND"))
  (pad "156" smd rect (at 35.04 -20.5 270) (size 0.2 0.7) (layers "F.Cu" "F.Mask" "F.Paste") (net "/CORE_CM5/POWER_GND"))
  (pad "157" smd rect (at 31.96 -20.1 270) (size 0.2 0.7) (layers "F.Cu" "F.Mask" "F.Paste") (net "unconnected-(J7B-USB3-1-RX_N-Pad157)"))
  (pad "158" smd rect (at 35.04 -20.1 270) (size 0.2 0.7) (layers "F.Cu" "F.Mask" "F.Paste") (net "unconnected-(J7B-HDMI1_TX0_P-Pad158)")
   (die_length 4.75))
  (pad "159" smd rect (at 31.96 -19.7 270) (size 0.2 0.7) (layers "F.Cu" "F.Mask" "F.Paste") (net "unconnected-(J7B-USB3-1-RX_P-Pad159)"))
  (pad "160" smd rect (at 35.04 -19.7 270) (size 0.2 0.7) (layers "F.Cu" "F.Mask" "F.Paste") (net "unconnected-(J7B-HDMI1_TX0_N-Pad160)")
   (die_length 4.76))
  (pad "161" smd rect (at 31.96 -19.3 270) (size 0.2 0.7) (layers "F.Cu" "F.Mask" "F.Paste") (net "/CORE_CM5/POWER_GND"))
  (pad "162" smd rect (at 35.04 -19.3 270) (size 0.2 0.7) (layers "F.Cu" "F.Mask" "F.Paste") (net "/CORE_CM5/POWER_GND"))
  (pad "163" smd rect (at 31.96 -18.9 270) (size 0.2 0.7) (layers "F.Cu" "F.Mask" "F.Paste") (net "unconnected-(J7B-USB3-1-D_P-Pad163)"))
  (pad "164" smd rect (at 35.04 -18.9 270) (size 0.2 0.7) (layers "F.Cu" "F.Mask" "F.Paste") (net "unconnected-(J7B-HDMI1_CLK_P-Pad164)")
   (die_length 2.99))
  (pad "165" smd rect (at 31.96 -18.5 270) (size 0.2 0.7) (layers "F.Cu" "F.Mask" "F.Paste") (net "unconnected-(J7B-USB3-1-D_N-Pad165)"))
  (pad "166" smd rect (at 35.04 -18.5 270) (size 0.2 0.7) (layers "F.Cu" "F.Mask" "F.Paste") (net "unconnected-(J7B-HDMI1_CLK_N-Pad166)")
   (die_length 2.99))
  (pad "167" smd rect (at 31.96 -18.1 270) (size 0.2 0.7) (layers "F.Cu" "F.Mask" "F.Paste") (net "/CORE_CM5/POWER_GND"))
  (pad "168" smd rect (at 35.04 -18.1 270) (size 0.2 0.7) (layers "F.Cu" "F.Mask" "F.Paste") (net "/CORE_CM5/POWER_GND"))
  (pad "169" smd rect (at 31.96 -17.7 270) (size 0.2 0.7) (layers "F.Cu" "F.Mask" "F.Paste") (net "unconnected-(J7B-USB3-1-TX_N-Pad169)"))
  (pad "170" smd rect (at 35.04 -17.7 270) (size 0.2 0.7) (layers "F.Cu" "F.Mask" "F.Paste") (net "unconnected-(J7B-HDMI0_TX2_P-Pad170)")
   (die_length 0.25))
  (pad "171" smd rect (at 31.96 -17.3 270) (size 0.2 0.7) (layers "F.Cu" "F.Mask" "F.Paste") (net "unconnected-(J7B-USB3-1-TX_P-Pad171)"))
  (pad "172" smd rect (at 35.04 -17.3 270) (size 0.2 0.7) (layers "F.Cu" "F.Mask" "F.Paste") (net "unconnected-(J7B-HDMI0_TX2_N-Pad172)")
   (die_length 0.25))
  (pad "173" smd rect (at 31.96 -16.9 270) (size 0.2 0.7) (layers "F.Cu" "F.Mask" "F.Paste") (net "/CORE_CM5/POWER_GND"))
  (pad "174" smd rect (at 35.04 -16.9 270) (size 0.2 0.7) (layers "F.Cu" "F.Mask" "F.Paste") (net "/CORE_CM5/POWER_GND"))
  (pad "175" smd rect (at 31.96 -16.5 270) (size 0.2 0.7) (layers "F.Cu" "F.Mask" "F.Paste") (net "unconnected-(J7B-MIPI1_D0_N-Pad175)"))
  (pad "176" smd rect (at 35.04 -16.5 270) (size 0.2 0.7) (layers "F.Cu" "F.Mask" "F.Paste") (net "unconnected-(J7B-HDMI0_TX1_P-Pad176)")
   (die_length 5.18))
  (pad "177" smd rect (at 31.96 -16.1 270) (size 0.2 0.7) (layers "F.Cu" "F.Mask" "F.Paste") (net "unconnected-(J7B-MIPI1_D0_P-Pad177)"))
  (pad "178" smd rect (at 35.04 -16.1 270) (size 0.2 0.7) (layers "F.Cu" "F.Mask" "F.Paste") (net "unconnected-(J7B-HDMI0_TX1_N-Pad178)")
   (die_length 5.18))
  (pad "179" smd rect (at 31.96 -15.7 270) (size 0.2 0.7) (layers "F.Cu" "F.Mask" "F.Paste") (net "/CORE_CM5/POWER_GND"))
  (pad "180" smd rect (at 35.04 -15.7 270) (size 0.2 0.7) (layers "F.Cu" "F.Mask" "F.Paste") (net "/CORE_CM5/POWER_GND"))
  (pad "181" smd rect (at 31.96 -15.3 270) (size 0.2 0.7) (layers "F.Cu" "F.Mask" "F.Paste") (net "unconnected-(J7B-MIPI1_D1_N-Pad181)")
   (die_length 1.06))
  (pad "182" smd rect (at 35.04 -15.3 270) (size 0.2 0.7) (layers "F.Cu" "F.Mask" "F.Paste") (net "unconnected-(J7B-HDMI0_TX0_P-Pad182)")
   (die_length 0.18))
  (pad "183" smd rect (at 31.96 -14.9 270) (size 0.2 0.7) (layers "F.Cu" "F.Mask" "F.Paste") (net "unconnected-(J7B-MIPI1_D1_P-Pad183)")
   (die_length 1.05))
  (pad "184" smd rect (at 35.04 -14.9 270) (size 0.2 0.7) (layers "F.Cu" "F.Mask" "F.Paste") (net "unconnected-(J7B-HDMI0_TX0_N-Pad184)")
   (die_length 0.18))
  (pad "185" smd rect (at 31.96 -14.5 270) (size 0.2 0.7) (layers "F.Cu" "F.Mask" "F.Paste") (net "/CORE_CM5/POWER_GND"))
  (pad "186" smd rect (at 35.04 -14.5 270) (size 0.2 0.7) (layers "F.Cu" "F.Mask" "F.Paste") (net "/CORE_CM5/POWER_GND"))
  (pad "187" smd rect (at 31.96 -14.1 270) (size 0.2 0.7) (layers "F.Cu" "F.Mask" "F.Paste") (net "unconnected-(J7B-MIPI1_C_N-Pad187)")
   (die_length 1.28))
  (pad "188" smd rect (at 35.04 -14.1 270) (size 0.2 0.7) (layers "F.Cu" "F.Mask" "F.Paste") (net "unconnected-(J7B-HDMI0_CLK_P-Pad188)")
   (die_length 0.91))
  (pad "189" smd rect (at 31.96 -13.7 270) (size 0.2 0.7) (layers "F.Cu" "F.Mask" "F.Paste") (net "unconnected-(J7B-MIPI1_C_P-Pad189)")
   (die_length 1.27))
  (pad "190" smd rect (at 35.04 -13.7 270) (size 0.2 0.7) (layers "F.Cu" "F.Mask" "F.Paste") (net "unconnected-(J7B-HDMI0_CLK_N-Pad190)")
   (die_length 0.91))
  (pad "191" smd rect (at 31.96 -13.3 270) (size 0.2 0.7) (layers "F.Cu" "F.Mask" "F.Paste") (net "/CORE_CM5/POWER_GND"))
  (pad "192" smd rect (at 35.04 -13.3 270) (size 0.2 0.7) (layers "F.Cu" "F.Mask" "F.Paste") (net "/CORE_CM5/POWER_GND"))
  (pad "193" smd rect (at 31.96 -12.9 270) (size 0.2 0.7) (layers "F.Cu" "F.Mask" "F.Paste") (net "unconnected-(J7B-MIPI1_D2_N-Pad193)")
   (die_length 0.83))
  (pad "194" smd rect (at 35.04 -12.9 270) (size 0.2 0.7) (layers "F.Cu" "F.Mask" "F.Paste") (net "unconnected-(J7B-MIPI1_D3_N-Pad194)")
   (die_length 3.79))
  (pad "195" smd rect (at 31.96 -12.5 270) (size 0.2 0.7) (layers "F.Cu" "F.Mask" "F.Paste") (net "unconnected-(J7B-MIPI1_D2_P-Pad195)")
   (die_length 0.84))
  (pad "196" smd rect (at 35.04 -12.5 270) (size 0.2 0.7) (layers "F.Cu" "F.Mask" "F.Paste") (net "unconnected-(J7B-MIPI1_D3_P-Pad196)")
   (die_length 3.79))
  (pad "197" smd rect (at 31.96 -12.1 270) (size 0.2 0.7) (layers "F.Cu" "F.Mask" "F.Paste") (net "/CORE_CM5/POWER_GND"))
  (pad "198" smd rect (at 35.04 -12.1 270) (size 0.2 0.7) (layers "F.Cu" "F.Mask" "F.Paste") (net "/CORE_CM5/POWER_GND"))
  (pad "199" smd rect (at 31.96 -11.7 270) (size 0.2 0.7) (layers "F.Cu" "F.Mask" "F.Paste") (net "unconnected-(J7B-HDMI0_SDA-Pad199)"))
  (pad "200" smd rect (at 35.04 -11.7 270) (size 0.2 0.7) (layers "F.Cu" "F.Mask" "F.Paste") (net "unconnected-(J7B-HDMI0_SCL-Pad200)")))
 (gr_line (start 5 70) (end 100 70) (stroke (width 0.05) (type default)) (layer "Edge.Cuts"))
 (gr_line (start 5 145) (end 5 70) (stroke (width 0.05) (type default)) (layer "Edge.Cuts"))
 (gr_line (start 100 70) (end 100 145) (stroke (width 0.05) (type default)) (layer "Edge.Cuts"))
 (gr_line (start 100 145) (end 5 145) (stroke (width 0.05) (type default)) (layer "Edge.Cuts"))
 (segment (start 32.96 99.1) (end 30 99.1) (width 0.127) (layer "F.Cu") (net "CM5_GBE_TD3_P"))
 (via (at 30 99.1) (size 0.5) (drill 0.3) (layers "F.Cu" "B.Cu") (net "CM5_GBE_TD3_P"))
 (segment (start 30 99.1) (end 10 90) (width 0.127) (layer "B.Cu") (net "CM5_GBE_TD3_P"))
 (segment (start 80 72) (end 80 90) (width 0.127) (layer "F.Cu") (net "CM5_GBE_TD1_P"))
 (segment (start 36.04 99.1) (end 40 97.5) (width 0.127) (layer "F.Cu") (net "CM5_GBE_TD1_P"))
 (segment (start 40 72) (end 80 72) (width 0.127) (layer "F.Cu") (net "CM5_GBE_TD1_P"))
 (segment (start 80 90) (end 90 90) (width 0.127) (layer "F.Cu") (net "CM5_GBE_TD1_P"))
 (via (at 40 97.5) (size 0.5) (drill 0.3) (layers "F.Cu" "B.Cu") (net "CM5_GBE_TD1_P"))
 (via (at 40 72) (size 0.5) (drill 0.3) (layers "F.Cu" "B.Cu") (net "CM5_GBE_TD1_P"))
 (segment (start 40 97.5) (end 40 72) (width 0.127) (layer "B.Cu") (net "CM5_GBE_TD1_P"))
 (segment (start 32.96 99.5) (end 28 99.5) (width 0.127) (layer "F.Cu") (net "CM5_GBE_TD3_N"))
 (via (at 28 99.5) (size 0.5) (drill 0.3) (layers "F.Cu" "B.Cu") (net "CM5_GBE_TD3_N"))
 (segment (start 28 99.5) (end 8 92) (width 0.127) (layer "B.Cu") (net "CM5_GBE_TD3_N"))
 (segment (start 78.5 72.5) (end 78.5 92) (width 0.127) (layer "F.Cu") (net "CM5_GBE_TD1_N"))
 (segment (start 42 72.5) (end 78.5 72.5) (width 0.127) (layer "F.Cu") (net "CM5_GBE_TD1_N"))
 (segment (start 78.5 92) (end 92 92) (width 0.127) (layer "F.Cu") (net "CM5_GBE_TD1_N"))
 (segment (start 36.04 99.5) (end 42 100.3) (width 0.127) (layer "F.Cu") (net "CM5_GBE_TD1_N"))
 (via (at 42 100.3) (size 0.5) (drill 0.3) (layers "F.Cu" "B.Cu") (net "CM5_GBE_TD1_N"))
 (via (at 42 72.5) (size 0.5) (drill 0.3) (layers "F.Cu" "B.Cu") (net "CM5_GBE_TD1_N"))
 (segment (start 42 100.3) (end 42 72.5) (width 0.127) (layer "B.Cu") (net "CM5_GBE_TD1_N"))
 (segment (start 32.96 100.3) (end 26 100.3) (width 0.127) (layer "F.Cu") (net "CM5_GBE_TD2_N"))
 (via (at 26 100.3) (size 0.5) (drill 0.3) (layers "F.Cu" "B.Cu") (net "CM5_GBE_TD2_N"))
 (segment (start 26 100.3) (end 6 94) (width 0.127) (layer "B.Cu") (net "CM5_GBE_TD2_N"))
 (segment (start 36.04 100.3) (end 44 101.899999) (width 0.127) (layer "F.Cu") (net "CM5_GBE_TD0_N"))
 (segment (start 77 73) (end 77 94) (width 0.127) (layer "F.Cu") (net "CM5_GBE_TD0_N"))
 (segment (start 77 94) (end 94 94) (width 0.127) (layer "F.Cu") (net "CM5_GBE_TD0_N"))
 (segment (start 44 73) (end 77 73) (width 0.127) (layer "F.Cu") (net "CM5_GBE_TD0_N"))
 (via (at 44 101.899999) (size 0.5) (drill 0.3) (layers "F.Cu" "B.Cu") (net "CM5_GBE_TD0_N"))
 (via (at 44 73) (size 0.5) (drill 0.3) (layers "F.Cu" "B.Cu") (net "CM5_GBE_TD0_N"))
 (segment (start 44 101.899999) (end 44 73) (width 0.127) (layer "B.Cu") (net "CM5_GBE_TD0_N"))
 (segment (start 32.96 100.7) (end 24 100.7) (width 0.127) (layer "F.Cu") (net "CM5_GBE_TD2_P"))
 (via (at 24 100.7) (size 0.5) (drill 0.3) (layers "F.Cu" "B.Cu") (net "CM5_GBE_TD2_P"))
 (segment (start 24 100.7) (end 4 96) (width 0.127) (layer "B.Cu") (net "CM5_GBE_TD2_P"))
 (segment (start 75.5 96) (end 96 96) (width 0.127) (layer "F.Cu") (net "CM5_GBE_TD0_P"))
 (segment (start 36.04 100.7) (end 46 103.1) (width 0.127) (layer "F.Cu") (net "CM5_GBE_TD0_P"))
 (segment (start 46 73.5) (end 75.5 73.5) (width 0.127) (layer "F.Cu") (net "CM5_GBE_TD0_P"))
 (segment (start 75.5 73.5) (end 75.5 96) (width 0.127) (layer "F.Cu") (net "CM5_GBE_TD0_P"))
 (via (at 46 103.1) (size 0.5) (drill 0.3) (layers "F.Cu" "B.Cu") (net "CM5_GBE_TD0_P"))
 (via (at 46 73.5) (size 0.5) (drill 0.3) (layers "F.Cu" "B.Cu") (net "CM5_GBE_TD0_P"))
 (segment (start 46 103.1) (end 46 73.5) (width 0.127) (layer "B.Cu") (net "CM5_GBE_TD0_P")))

